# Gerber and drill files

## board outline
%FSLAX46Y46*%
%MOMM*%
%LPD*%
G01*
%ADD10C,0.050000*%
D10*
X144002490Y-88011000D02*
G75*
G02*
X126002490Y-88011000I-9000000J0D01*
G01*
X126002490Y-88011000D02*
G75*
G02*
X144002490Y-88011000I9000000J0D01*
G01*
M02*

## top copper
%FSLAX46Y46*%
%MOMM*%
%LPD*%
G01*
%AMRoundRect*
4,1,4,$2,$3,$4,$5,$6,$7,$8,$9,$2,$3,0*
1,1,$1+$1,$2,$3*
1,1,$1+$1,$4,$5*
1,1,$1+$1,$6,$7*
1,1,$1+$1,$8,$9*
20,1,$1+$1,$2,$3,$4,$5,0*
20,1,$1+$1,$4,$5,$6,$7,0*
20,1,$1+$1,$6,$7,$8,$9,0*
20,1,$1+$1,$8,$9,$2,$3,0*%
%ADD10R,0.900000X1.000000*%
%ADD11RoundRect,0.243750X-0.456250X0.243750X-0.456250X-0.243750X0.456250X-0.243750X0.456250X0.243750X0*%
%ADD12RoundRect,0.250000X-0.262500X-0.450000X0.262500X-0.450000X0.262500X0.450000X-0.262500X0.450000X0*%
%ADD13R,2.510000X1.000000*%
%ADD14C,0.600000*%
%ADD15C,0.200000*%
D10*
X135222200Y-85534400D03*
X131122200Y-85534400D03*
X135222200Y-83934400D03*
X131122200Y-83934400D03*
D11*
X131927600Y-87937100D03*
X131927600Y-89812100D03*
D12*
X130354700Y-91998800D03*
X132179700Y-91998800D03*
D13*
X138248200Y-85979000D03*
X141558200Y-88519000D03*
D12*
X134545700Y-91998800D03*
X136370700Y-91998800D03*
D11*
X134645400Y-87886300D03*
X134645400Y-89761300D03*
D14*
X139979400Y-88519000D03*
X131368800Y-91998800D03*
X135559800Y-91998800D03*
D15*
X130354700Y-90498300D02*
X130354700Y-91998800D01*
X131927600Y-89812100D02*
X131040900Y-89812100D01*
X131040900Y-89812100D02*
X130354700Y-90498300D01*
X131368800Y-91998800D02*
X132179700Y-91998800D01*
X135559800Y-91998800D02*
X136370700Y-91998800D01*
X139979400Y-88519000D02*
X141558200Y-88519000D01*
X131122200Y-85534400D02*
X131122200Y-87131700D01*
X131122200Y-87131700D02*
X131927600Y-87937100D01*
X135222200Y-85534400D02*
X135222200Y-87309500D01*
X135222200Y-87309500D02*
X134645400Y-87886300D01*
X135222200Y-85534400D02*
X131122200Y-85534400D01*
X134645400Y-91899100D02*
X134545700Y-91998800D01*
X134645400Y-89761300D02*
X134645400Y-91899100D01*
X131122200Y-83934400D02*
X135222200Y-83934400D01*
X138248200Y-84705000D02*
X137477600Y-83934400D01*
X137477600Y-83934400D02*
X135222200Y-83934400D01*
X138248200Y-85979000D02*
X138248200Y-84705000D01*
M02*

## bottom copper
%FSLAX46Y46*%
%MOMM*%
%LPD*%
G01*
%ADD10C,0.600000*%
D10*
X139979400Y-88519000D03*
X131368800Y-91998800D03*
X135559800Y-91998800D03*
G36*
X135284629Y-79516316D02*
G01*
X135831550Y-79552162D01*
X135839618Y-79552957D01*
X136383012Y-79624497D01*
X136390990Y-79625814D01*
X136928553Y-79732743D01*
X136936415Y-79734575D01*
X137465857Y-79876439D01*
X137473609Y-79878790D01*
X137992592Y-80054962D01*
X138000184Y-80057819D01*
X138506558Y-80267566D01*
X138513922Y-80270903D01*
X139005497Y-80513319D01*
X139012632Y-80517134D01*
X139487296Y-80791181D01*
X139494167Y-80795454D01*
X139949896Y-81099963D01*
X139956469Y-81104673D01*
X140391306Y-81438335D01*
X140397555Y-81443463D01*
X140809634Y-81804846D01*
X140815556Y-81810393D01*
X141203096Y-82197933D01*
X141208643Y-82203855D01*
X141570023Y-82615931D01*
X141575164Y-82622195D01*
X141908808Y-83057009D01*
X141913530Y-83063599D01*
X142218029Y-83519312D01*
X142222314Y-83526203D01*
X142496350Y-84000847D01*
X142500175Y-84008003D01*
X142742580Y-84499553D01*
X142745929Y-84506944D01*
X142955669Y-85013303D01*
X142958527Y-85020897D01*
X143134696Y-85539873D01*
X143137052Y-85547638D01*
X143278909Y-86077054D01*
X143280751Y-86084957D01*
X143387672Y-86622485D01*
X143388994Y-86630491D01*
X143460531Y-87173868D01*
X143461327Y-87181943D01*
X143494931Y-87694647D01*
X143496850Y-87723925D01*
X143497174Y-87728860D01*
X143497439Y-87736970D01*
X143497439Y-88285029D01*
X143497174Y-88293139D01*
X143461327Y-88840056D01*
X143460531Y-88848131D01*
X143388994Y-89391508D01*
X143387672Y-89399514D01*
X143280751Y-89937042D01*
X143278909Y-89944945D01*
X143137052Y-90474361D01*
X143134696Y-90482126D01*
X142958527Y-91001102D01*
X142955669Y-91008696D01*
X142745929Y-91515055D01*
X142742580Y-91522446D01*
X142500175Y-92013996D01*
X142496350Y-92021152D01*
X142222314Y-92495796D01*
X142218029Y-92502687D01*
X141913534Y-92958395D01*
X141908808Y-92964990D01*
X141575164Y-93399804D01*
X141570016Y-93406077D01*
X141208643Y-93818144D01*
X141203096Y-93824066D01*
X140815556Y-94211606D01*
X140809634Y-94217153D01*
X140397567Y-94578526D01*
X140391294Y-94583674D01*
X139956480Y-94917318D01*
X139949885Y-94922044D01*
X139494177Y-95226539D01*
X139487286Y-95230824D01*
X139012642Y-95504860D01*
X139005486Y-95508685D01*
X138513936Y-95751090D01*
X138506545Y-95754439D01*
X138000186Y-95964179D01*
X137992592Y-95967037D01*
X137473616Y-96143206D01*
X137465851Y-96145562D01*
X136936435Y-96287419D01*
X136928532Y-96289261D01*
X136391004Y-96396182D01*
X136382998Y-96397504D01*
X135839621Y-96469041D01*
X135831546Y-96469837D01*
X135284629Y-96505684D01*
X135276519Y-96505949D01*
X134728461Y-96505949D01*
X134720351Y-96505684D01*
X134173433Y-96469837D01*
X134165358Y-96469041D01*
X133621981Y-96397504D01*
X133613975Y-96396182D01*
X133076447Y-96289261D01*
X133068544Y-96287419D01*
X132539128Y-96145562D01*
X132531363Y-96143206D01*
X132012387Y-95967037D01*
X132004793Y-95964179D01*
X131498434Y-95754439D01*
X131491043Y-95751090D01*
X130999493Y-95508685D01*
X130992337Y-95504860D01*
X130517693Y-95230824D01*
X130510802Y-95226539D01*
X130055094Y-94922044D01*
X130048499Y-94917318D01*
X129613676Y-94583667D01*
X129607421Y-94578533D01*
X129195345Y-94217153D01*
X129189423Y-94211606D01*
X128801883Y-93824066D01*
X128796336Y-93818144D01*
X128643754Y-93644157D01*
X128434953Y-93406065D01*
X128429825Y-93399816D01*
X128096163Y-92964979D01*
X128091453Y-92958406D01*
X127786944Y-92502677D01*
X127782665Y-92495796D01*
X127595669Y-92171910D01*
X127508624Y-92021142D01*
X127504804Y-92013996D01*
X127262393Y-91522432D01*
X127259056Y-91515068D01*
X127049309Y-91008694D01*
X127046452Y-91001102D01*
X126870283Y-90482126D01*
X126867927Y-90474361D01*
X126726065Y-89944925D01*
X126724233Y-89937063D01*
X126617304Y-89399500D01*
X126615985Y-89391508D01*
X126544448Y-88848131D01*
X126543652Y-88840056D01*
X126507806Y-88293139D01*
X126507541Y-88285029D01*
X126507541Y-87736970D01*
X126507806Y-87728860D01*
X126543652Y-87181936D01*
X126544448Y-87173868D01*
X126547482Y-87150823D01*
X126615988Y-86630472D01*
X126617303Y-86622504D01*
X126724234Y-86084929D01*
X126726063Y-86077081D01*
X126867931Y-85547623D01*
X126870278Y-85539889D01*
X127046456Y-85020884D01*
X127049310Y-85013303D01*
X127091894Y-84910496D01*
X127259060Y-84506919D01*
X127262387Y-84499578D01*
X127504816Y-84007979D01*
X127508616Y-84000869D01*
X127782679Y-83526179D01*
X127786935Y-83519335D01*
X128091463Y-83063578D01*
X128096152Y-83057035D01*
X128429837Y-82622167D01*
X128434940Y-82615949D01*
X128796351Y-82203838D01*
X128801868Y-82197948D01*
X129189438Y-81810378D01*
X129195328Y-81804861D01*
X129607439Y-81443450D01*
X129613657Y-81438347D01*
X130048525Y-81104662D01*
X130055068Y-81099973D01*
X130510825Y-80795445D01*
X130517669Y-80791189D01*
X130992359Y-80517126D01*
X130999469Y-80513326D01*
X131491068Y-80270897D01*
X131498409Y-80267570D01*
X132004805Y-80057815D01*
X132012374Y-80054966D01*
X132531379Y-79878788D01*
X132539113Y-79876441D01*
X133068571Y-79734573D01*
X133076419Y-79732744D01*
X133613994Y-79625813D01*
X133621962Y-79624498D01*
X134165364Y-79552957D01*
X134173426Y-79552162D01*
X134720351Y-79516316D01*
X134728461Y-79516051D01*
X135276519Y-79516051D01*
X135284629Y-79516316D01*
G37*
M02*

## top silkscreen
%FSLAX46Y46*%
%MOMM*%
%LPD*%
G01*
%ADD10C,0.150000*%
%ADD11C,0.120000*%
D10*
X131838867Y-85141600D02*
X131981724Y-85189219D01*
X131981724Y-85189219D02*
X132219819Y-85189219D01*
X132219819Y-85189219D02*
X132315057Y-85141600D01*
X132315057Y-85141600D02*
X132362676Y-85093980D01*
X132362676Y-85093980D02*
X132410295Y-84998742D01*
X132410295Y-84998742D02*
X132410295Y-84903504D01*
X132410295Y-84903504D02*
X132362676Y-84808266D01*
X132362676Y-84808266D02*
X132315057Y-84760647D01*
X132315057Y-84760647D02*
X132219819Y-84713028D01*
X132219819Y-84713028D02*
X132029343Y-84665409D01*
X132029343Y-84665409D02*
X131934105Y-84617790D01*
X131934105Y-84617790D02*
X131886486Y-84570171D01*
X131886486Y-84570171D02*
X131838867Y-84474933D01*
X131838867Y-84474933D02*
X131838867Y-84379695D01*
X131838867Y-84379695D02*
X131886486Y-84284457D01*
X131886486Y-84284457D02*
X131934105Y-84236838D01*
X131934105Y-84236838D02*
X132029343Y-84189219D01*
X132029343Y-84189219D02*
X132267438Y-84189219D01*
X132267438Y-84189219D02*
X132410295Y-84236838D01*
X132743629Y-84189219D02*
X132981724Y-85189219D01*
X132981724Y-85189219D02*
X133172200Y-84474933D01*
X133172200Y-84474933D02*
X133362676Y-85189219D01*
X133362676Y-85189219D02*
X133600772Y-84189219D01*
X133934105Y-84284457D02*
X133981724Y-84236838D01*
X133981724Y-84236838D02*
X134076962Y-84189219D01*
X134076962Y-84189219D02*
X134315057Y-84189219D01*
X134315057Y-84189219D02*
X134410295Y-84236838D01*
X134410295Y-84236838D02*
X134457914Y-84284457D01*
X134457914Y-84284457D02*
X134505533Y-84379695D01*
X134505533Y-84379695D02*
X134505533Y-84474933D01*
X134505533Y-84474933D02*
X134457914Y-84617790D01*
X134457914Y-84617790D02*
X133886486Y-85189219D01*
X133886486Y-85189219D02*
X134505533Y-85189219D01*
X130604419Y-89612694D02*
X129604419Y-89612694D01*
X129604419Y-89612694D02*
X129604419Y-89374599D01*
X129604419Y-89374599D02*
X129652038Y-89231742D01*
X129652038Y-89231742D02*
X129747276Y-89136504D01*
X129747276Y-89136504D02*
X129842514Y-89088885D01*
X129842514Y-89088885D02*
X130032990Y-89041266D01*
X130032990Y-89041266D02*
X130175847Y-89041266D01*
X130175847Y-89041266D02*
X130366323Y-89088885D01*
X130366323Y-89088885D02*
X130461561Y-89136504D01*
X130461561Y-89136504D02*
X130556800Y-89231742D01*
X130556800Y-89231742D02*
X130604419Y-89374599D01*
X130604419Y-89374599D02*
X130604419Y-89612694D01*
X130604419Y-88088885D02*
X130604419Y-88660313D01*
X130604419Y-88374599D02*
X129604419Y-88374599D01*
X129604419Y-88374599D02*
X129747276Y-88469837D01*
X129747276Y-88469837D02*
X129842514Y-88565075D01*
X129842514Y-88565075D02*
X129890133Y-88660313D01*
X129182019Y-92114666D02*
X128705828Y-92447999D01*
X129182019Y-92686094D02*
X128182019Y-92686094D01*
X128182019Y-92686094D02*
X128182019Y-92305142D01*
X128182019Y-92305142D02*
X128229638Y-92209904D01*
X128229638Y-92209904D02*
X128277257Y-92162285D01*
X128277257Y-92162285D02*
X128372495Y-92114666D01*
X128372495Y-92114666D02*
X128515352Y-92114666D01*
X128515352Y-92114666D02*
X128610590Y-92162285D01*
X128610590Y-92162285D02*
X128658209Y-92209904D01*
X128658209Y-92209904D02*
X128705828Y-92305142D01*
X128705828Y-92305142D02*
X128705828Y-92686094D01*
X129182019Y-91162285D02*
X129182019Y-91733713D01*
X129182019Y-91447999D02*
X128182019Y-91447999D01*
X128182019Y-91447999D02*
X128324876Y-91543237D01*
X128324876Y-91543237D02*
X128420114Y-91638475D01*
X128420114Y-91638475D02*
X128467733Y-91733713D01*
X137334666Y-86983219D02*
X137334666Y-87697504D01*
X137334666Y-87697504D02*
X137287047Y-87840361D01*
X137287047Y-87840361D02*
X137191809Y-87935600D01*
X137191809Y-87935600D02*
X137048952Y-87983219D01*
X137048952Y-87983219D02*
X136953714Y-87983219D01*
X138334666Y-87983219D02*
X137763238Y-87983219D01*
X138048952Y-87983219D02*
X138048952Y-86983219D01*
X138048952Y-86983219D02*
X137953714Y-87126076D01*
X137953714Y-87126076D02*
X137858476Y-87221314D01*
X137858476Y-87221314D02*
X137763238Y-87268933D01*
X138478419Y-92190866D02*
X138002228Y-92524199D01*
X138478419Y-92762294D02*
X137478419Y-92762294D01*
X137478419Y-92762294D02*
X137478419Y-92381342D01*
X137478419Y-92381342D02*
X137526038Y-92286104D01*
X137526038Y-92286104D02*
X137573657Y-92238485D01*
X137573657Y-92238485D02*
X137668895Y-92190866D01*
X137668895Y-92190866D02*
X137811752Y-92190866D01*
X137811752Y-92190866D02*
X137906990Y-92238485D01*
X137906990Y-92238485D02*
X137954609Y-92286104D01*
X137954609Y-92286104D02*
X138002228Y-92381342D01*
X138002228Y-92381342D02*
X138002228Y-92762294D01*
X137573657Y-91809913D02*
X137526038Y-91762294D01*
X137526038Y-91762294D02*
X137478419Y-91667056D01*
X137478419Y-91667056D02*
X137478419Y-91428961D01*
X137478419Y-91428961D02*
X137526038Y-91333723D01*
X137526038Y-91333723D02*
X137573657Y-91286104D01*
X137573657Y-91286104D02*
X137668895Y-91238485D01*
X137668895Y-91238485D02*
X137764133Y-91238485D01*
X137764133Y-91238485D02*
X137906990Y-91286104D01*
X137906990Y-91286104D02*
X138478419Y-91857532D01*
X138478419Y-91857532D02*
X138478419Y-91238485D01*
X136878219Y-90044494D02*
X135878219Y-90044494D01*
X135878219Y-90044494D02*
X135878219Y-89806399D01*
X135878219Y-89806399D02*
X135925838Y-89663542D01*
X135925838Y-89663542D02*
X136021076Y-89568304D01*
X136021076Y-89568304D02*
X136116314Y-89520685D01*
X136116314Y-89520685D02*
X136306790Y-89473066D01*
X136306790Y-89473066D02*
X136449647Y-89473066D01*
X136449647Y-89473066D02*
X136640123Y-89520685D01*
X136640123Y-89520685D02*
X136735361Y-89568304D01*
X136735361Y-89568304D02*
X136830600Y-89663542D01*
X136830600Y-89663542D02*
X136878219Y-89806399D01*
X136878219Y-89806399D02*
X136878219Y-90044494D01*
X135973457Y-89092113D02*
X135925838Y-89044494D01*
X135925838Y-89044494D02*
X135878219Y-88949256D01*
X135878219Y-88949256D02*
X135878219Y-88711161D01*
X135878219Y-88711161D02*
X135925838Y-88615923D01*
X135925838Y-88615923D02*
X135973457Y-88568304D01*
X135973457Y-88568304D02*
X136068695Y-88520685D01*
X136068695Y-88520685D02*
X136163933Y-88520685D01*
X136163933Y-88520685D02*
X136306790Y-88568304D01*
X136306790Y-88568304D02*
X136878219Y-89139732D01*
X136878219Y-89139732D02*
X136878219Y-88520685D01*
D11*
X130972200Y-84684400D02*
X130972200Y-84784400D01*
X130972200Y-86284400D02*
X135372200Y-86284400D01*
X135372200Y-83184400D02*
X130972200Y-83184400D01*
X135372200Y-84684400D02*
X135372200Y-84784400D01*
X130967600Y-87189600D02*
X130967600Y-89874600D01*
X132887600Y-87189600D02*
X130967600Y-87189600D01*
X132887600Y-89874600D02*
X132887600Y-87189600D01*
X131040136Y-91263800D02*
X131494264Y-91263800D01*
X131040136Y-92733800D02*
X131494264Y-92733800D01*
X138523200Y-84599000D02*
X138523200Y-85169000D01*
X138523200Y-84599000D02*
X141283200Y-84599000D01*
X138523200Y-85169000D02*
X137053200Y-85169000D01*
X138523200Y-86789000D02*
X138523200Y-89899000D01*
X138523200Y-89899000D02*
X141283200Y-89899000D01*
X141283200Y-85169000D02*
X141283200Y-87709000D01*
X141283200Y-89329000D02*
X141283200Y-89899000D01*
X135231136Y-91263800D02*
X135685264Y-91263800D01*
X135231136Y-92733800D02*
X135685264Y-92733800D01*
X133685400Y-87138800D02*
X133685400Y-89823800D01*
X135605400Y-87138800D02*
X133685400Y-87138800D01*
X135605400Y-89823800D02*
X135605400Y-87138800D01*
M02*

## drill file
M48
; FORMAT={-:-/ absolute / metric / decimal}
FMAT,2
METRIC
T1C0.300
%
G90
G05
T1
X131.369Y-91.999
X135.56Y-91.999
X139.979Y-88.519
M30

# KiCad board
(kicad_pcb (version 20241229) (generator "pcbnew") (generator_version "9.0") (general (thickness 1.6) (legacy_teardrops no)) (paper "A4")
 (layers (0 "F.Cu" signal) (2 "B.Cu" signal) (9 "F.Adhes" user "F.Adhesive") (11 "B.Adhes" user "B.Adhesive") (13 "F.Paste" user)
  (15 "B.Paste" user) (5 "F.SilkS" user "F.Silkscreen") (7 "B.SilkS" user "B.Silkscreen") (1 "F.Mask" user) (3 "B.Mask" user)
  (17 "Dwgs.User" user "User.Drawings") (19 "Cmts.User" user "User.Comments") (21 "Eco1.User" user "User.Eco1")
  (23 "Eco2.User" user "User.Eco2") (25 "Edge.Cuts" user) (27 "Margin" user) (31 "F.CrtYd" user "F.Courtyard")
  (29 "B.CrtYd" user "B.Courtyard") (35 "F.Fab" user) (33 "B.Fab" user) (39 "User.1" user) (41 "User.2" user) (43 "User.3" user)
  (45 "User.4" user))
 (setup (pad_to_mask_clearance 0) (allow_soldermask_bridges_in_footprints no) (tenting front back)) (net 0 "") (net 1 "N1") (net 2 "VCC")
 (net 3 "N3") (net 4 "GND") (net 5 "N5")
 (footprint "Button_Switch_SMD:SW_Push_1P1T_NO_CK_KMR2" (layer "F.Cu") (at 133.1722 84.7344 180)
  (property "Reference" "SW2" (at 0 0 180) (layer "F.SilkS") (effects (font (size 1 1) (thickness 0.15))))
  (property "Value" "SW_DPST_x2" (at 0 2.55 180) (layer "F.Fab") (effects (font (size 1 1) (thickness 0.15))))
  (fp_line (start 2.2 0.05) (end 2.2 -0.05) (stroke (width 0.12) (type solid)) (layer "F.SilkS"))
  (fp_line (start 2.2 -1.55) (end -2.2 -1.55) (stroke (width 0.12) (type solid)) (layer "F.SilkS"))
  (fp_line (start -2.2 1.55) (end 2.2 1.55) (stroke (width 0.12) (type solid)) (layer "F.SilkS"))
  (fp_line (start -2.2 0.05) (end -2.2 -0.05) (stroke (width 0.12) (type solid)) (layer "F.SilkS"))
  (pad "1" smd rect (at -2.05 -0.8 180) (size 0.9 1) (layers "F.Cu" "F.Mask" "F.Paste") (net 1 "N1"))
  (pad "1" smd rect (at 2.05 -0.8 180) (size 0.9 1) (layers "F.Cu" "F.Mask" "F.Paste") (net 1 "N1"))
  (pad "2" smd rect (at -2.05 0.8 180) (size 0.9 1) (layers "F.Cu" "F.Mask" "F.Paste") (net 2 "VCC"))
  (pad "2" smd rect (at 2.05 0.8 180) (size 0.9 1) (layers "F.Cu" "F.Mask" "F.Paste") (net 2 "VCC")))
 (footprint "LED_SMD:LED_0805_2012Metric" (layer "F.Cu") (at 131.9276 88.8746 -90)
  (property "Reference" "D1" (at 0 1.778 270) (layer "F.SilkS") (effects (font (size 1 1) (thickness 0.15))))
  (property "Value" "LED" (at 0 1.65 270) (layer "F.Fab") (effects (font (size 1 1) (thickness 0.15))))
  (fp_line (start -1.685 0.96) (end 1 0.96) (stroke (width 0.12) (type solid)) (layer "F.SilkS"))
  (fp_line (start -1.685 -0.96) (end -1.685 0.96) (stroke (width 0.12) (type solid)) (layer "F.SilkS"))
  (fp_line (start 1 -0.96) (end -1.685 -0.96) (stroke (width 0.12) (type solid)) (layer "F.SilkS"))
  (pad "1" smd roundrect (at -0.9375 0 270) (size 0.975 1.4) (layers "F.Cu" "F.Mask" "F.Paste") (roundrect_rratio 0.25) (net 1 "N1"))
  (pad "2" smd roundrect (at 0.9375 0 270) (size 0.975 1.4) (layers "F.Cu" "F.Mask" "F.Paste") (roundrect_rratio 0.25) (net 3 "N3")))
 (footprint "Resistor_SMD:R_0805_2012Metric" (layer "F.Cu") (at 131.2672 91.9988)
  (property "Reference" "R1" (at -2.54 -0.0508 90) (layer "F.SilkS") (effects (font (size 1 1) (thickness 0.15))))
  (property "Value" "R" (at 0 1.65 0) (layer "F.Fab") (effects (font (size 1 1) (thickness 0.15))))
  (fp_line (start -0.227064 -0.735) (end 0.227064 -0.735) (stroke (width 0.12) (type solid)) (layer "F.SilkS"))
  (fp_line (start -0.227064 0.735) (end 0.227064 0.735) (stroke (width 0.12) (type solid)) (layer "F.SilkS"))
  (pad "1" smd roundrect (at -0.9125 0) (size 1.025 1.4) (layers "F.Cu" "F.Mask" "F.Paste") (roundrect_rratio 0.243902) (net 3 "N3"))
  (pad "2" smd roundrect (at 0.9125 0) (size 1.025 1.4) (layers "F.Cu" "F.Mask" "F.Paste") (roundrect_rratio 0.243902) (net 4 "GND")))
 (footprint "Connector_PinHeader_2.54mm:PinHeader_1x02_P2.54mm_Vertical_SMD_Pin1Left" (layer "F.Cu") (at 139.9032 87.249)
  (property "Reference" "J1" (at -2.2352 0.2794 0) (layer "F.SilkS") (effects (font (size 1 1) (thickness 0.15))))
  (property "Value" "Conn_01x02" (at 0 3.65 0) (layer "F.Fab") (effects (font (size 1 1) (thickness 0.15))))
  (fp_line (start -1.38 -2.65) (end -1.38 -2.08) (stroke (width 0.12) (type solid)) (layer "F.SilkS"))
  (fp_line (start -1.38 -2.65) (end 1.38 -2.65) (stroke (width 0.12) (type solid)) (layer "F.SilkS"))
  (fp_line (start -1.38 -2.08) (end -2.85 -2.08) (stroke (width 0.12) (type solid)) (layer "F.SilkS"))
  (fp_line (start -1.38 -0.46) (end -1.38 2.65) (stroke (width 0.12) (type solid)) (layer "F.SilkS"))
  (fp_line (start -1.38 2.65) (end 1.38 2.65) (stroke (width 0.12) (type solid)) (layer "F.SilkS"))
  (fp_line (start 1.38 -2.08) (end 1.38 0.46) (stroke (width 0.12) (type solid)) (layer "F.SilkS"))
  (fp_line (start 1.38 2.08) (end 1.38 2.65) (stroke (width 0.12) (type solid)) (layer "F.SilkS"))
  (pad "1" smd rect (at -1.655 -1.27) (size 2.51 1) (layers "F.Cu" "F.Mask" "F.Paste") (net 2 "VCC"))
  (pad "2" smd rect (at 1.655 1.27) (size 2.51 1) (layers "F.Cu" "F.Mask" "F.Paste") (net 4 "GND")))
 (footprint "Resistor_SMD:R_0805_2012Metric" (layer "F.Cu") (at 135.4582 91.9988)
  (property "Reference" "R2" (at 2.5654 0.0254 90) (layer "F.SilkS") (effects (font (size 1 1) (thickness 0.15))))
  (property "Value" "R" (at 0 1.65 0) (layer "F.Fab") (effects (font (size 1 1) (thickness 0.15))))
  (fp_line (start -0.227064 -0.735) (end 0.227064 -0.735) (stroke (width 0.12) (type solid)) (layer "F.SilkS"))
  (fp_line (start -0.227064 0.735) (end 0.227064 0.735) (stroke (width 0.12) (type solid)) (layer "F.SilkS"))
  (pad "1" smd roundrect (at -0.9125 0) (size 1.025 1.4) (layers "F.Cu" "F.Mask" "F.Paste") (roundrect_rratio 0.243902) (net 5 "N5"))
  (pad "2" smd roundrect (at 0.9125 0) (size 1.025 1.4) (layers "F.Cu" "F.Mask" "F.Paste") (roundrect_rratio 0.243902) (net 4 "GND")))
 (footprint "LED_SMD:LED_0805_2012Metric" (layer "F.Cu") (at 134.6454 88.8238 -90)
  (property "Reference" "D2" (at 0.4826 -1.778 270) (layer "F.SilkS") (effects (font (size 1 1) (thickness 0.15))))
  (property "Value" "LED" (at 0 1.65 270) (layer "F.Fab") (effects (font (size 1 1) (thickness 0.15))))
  (fp_line (start -1.685 0.96) (end 1 0.96) (stroke (width 0.12) (type solid)) (layer "F.SilkS"))
  (fp_line (start -1.685 -0.96) (end -1.685 0.96) (stroke (width 0.12) (type solid)) (layer "F.SilkS"))
  (fp_line (start 1 -0.96) (end -1.685 -0.96) (stroke (width 0.12) (type solid)) (layer "F.SilkS"))
  (pad "1" smd roundrect (at -0.9375 0 270) (size 0.975 1.4) (layers "F.Cu" "F.Mask" "F.Paste") (roundrect_rratio 0.25) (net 1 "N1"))
  (pad "2" smd roundrect (at 0.9375 0 270) (size 0.975 1.4) (layers "F.Cu" "F.Mask" "F.Paste") (roundrect_rratio 0.25) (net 5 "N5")))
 (gr_circle (center 135.00249 88.011) (end 144.00249 88.011) (stroke (width 0.05) (type solid)) (fill no) (layer "Edge.Cuts"))
 (segment (start 130.3547 90.4983) (end 130.3547 91.9988) (width 0.2) (layer "F.Cu") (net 3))
 (segment (start 131.9276 89.8121) (end 131.0409 89.8121) (width 0.2) (layer "F.Cu") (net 3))
 (segment (start 131.0409 89.8121) (end 130.3547 90.4983) (width 0.2) (layer "F.Cu") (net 3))
 (segment (start 131.3688 91.9988) (end 132.1797 91.9988) (width 0.2) (layer "F.Cu") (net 4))
 (segment (start 135.5598 91.9988) (end 136.3707 91.9988) (width 0.2) (layer "F.Cu") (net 4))
 (segment (start 139.9794 88.519) (end 141.5582 88.519) (width 0.2) (layer "F.Cu") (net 4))
 (via (at 139.9794 88.519) (size 0.6) (drill 0.3) (layers "F.Cu" "B.Cu") (free yes) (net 4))
 (via (at 131.3688 91.9988) (size 0.6) (drill 0.3) (layers "F.Cu" "B.Cu") (free yes) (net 4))
 (via (at 135.5598 91.9988) (size 0.6) (drill 0.3) (layers "F.Cu" "B.Cu") (free yes) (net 4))
 (segment (start 131.1222 85.5344) (end 131.1222 87.1317) (width 0.2) (layer "F.Cu") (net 1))
 (segment (start 131.1222 87.1317) (end 131.9276 87.9371) (width 0.2) (layer "F.Cu") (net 1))
 (segment (start 135.2222 85.5344) (end 135.2222 87.3095) (width 0.2) (layer "F.Cu") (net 1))
 (segment (start 135.2222 87.3095) (end 134.6454 87.8863) (width 0.2) (layer "F.Cu") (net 1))
 (segment (start 135.2222 85.5344) (end 131.1222 85.5344) (width 0.2) (layer "F.Cu") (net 1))
 (segment (start 134.6454 91.8991) (end 134.5457 91.9988) (width 0.2) (layer "F.Cu") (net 5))
 (segment (start 134.6454 89.7613) (end 134.6454 91.8991) (width 0.2) (layer "F.Cu") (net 5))
 (segment (start 131.1222 83.9344) (end 135.2222 83.9344) (width 0.2) (layer "F.Cu") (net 2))
 (segment (start 138.2482 84.705) (end 137.4776 83.9344) (width 0.2) (layer "F.Cu") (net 2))
 (segment (start 137.4776 83.9344) (end 135.2222 83.9344) (width 0.2) (layer "F.Cu") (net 2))
 (segment (start 138.2482 85.979) (end 138.2482 84.705) (width 0.2) (layer "F.Cu") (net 2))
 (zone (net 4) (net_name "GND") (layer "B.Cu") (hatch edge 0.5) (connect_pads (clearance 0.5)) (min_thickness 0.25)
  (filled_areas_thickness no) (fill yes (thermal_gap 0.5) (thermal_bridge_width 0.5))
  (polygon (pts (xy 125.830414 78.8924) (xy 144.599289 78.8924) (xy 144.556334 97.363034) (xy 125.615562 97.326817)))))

